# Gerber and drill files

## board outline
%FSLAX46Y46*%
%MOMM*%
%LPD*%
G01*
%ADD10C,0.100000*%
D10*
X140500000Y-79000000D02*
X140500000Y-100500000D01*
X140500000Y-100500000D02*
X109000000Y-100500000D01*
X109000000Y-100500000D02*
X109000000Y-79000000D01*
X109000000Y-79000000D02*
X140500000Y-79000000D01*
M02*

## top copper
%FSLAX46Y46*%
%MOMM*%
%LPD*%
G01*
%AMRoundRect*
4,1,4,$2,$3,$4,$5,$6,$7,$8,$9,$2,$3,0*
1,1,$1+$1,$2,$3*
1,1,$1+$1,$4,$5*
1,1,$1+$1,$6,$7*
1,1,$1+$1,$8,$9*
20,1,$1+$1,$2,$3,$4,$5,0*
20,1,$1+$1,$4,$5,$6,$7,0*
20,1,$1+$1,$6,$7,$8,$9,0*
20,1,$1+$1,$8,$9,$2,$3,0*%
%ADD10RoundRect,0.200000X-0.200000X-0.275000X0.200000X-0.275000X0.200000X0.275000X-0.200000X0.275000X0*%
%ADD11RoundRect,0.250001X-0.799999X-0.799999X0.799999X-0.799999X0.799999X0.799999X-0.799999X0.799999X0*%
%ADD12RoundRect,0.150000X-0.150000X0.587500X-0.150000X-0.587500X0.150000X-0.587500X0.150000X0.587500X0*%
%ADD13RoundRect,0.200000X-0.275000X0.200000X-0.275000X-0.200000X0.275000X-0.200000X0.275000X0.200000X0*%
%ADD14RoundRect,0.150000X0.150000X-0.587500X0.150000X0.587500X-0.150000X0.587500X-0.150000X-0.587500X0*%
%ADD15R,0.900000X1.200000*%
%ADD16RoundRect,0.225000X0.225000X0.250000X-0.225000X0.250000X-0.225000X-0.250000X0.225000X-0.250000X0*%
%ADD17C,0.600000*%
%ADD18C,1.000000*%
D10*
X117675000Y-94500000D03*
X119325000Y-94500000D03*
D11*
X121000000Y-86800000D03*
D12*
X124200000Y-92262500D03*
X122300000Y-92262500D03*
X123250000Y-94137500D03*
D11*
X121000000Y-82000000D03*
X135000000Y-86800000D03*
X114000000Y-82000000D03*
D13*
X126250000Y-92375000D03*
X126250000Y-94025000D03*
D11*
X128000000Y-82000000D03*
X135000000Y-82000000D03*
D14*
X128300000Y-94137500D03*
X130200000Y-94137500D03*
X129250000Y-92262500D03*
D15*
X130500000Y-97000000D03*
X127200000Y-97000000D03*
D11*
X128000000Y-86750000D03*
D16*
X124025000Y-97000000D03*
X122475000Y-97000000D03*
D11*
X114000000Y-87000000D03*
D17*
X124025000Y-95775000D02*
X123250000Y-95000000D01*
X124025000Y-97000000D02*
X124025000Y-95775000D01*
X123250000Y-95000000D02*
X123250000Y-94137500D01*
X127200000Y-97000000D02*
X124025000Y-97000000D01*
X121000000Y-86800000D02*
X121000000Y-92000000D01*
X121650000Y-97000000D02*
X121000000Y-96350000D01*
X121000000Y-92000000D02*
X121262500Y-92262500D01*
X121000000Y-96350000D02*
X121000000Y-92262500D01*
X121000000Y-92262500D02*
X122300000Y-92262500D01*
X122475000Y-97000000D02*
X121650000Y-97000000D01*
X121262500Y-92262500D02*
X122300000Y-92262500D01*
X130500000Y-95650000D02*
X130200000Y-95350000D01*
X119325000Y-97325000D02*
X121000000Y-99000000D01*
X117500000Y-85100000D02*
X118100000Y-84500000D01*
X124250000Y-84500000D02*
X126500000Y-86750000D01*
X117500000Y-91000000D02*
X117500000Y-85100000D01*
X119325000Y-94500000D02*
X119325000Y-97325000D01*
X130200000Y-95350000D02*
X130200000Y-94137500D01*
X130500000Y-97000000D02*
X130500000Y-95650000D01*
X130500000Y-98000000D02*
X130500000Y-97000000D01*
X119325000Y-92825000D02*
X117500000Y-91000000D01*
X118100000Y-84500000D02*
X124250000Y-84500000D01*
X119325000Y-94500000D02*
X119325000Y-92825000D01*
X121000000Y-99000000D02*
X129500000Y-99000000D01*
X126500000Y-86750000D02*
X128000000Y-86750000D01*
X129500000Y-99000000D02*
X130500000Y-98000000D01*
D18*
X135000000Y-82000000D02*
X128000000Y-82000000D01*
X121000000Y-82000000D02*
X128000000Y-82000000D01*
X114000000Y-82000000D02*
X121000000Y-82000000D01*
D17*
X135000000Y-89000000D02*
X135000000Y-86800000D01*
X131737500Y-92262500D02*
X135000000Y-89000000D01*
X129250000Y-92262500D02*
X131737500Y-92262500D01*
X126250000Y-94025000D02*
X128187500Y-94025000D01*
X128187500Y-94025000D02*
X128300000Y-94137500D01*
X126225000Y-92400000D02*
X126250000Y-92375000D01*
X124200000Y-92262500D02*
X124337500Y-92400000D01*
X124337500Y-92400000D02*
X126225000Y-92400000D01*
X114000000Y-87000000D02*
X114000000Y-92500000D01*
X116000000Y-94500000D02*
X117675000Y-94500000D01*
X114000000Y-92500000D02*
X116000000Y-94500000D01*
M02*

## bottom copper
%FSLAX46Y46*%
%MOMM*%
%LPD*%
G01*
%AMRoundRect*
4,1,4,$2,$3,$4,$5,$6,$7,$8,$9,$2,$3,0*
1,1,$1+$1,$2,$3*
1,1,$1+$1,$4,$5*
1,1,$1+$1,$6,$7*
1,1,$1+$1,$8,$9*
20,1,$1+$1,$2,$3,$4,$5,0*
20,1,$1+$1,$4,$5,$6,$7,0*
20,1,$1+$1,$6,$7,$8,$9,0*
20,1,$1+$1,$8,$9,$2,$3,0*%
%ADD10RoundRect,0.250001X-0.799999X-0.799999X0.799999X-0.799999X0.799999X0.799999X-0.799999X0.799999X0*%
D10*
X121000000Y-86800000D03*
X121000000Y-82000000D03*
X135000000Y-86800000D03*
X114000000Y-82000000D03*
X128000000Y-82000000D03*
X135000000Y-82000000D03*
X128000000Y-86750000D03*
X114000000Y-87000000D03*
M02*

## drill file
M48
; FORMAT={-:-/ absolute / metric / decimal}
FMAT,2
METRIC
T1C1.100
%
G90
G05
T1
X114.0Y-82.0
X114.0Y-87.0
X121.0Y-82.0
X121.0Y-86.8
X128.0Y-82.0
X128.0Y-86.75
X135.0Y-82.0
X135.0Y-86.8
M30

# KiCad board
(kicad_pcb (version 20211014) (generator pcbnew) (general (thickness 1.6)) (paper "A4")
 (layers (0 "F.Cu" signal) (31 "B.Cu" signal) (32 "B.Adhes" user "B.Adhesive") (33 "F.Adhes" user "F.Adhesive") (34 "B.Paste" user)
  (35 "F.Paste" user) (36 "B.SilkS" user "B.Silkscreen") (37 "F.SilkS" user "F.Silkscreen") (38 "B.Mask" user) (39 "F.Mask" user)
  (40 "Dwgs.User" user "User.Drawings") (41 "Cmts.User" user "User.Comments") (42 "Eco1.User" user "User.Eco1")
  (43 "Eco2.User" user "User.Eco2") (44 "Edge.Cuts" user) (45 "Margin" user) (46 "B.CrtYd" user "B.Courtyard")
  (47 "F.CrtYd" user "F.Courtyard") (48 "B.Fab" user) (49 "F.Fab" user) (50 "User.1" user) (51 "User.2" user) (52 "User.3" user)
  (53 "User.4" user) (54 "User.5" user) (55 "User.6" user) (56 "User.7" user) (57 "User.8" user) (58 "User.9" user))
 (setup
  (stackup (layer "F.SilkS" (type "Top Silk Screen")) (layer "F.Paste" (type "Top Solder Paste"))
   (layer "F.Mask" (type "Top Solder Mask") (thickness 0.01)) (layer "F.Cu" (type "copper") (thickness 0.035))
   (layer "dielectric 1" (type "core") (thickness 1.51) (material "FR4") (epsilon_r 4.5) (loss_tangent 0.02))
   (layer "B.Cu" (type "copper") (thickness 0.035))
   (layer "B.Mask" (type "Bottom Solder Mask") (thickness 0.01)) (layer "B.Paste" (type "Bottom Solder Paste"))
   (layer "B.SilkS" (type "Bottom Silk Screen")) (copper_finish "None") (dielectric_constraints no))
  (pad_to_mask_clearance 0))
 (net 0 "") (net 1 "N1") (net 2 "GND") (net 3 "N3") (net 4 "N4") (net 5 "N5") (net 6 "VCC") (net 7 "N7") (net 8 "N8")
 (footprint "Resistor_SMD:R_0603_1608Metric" (layer "F.Cu") (at 118.5 94.5)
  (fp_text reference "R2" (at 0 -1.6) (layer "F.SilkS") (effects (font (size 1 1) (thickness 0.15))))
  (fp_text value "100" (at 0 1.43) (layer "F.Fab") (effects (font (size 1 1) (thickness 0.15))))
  (pad "1" smd roundrect (at -0.825 0) (size 0.8 0.95) (layers "F.Cu" "F.Paste" "F.Mask") (roundrect_rratio 0.25) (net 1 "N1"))
  (pad "2" smd roundrect (at 0.825 0) (size 0.8 0.95) (layers "F.Cu" "F.Paste" "F.Mask") (roundrect_rratio 0.25) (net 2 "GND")))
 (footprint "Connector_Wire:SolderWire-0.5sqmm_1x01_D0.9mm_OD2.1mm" (layer "F.Cu") (at 121 86.8)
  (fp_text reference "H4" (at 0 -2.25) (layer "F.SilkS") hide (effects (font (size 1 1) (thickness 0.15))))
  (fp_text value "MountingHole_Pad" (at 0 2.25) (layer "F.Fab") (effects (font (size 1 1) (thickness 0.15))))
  (pad "1" thru_hole roundrect (at 0 0) (size 2.1 2.1) (drill 1.1) (layers *.Cu *.Mask) (roundrect_rratio 0.119048) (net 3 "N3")))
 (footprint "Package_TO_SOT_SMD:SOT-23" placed (layer "F.Cu") (at 123.25 93.2 -90)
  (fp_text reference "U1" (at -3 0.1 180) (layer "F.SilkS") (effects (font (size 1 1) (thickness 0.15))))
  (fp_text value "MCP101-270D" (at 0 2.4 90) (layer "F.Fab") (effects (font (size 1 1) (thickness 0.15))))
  (pad "1" smd roundrect (at -0.9375 -0.95 270) (size 1.475 0.6) (layers "F.Cu" "F.Paste" "F.Mask") (roundrect_rratio 0.25) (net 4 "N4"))
  (pad "2" smd roundrect (at -0.9375 0.95 270) (size 1.475 0.6) (layers "F.Cu" "F.Paste" "F.Mask") (roundrect_rratio 0.25) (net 3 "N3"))
  (pad "3" smd roundrect (at 0.9375 0 270) (size 1.475 0.6) (layers "F.Cu" "F.Paste" "F.Mask") (roundrect_rratio 0.25) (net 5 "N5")))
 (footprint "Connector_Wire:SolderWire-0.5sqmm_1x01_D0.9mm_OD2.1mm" (layer "F.Cu") (at 121 82)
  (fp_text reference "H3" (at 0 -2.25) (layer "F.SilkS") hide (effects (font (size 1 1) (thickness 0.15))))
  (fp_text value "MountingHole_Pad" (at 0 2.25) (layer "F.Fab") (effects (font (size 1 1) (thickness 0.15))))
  (pad "1" thru_hole roundrect (at 0 0) (size 2.1 2.1) (drill 1.1) (layers *.Cu *.Mask) (roundrect_rratio 0.119048) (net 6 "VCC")))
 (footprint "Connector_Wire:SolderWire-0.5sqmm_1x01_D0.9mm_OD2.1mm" (layer "F.Cu") (at 135 86.8)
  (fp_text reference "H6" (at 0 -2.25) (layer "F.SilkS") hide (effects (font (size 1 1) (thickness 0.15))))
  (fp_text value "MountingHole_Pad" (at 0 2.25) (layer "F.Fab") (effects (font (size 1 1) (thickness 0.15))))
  (pad "1" thru_hole roundrect (at 0 0) (size 2.1 2.1) (drill 1.1) (layers *.Cu *.Mask) (roundrect_rratio 0.119048) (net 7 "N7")))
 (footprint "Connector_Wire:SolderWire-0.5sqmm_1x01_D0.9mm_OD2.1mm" (layer "F.Cu") (at 114 82)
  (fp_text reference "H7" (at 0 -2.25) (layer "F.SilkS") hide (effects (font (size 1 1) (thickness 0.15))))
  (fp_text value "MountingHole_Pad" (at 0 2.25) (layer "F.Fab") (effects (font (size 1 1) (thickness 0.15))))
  (pad "1" thru_hole roundrect (at 0 0) (size 2.1 2.1) (drill 1.1) (layers *.Cu *.Mask) (roundrect_rratio 0.119048) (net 6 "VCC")))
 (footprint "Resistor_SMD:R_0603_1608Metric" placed (layer "F.Cu") (at 126.25 93.2 -90)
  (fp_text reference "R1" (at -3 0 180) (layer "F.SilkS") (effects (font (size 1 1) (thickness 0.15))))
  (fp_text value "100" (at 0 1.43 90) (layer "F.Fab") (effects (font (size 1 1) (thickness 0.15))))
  (pad "1" smd roundrect (at -0.825 0 270) (size 0.8 0.95) (layers "F.Cu" "F.Paste" "F.Mask") (roundrect_rratio 0.25) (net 4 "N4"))
  (pad "2" smd roundrect (at 0.825 0 270) (size 0.8 0.95) (layers "F.Cu" "F.Paste" "F.Mask") (roundrect_rratio 0.25) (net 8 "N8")))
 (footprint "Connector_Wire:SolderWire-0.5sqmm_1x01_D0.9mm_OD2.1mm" (layer "F.Cu") (at 128 82)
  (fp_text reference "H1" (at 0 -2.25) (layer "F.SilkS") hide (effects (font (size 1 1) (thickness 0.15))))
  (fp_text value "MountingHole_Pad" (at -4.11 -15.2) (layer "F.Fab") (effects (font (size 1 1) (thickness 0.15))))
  (pad "1" thru_hole roundrect (at 0 0) (size 2.1 2.1) (drill 1.1) (layers *.Cu *.Mask) (roundrect_rratio 0.119048) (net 6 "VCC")))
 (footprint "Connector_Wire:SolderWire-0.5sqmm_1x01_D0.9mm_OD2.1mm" (layer "F.Cu") (at 135 82)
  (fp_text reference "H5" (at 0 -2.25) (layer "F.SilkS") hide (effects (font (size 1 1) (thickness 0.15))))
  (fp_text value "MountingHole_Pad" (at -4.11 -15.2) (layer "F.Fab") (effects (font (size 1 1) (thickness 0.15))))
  (pad "1" thru_hole roundrect (at 0 0) (size 2.1 2.1) (drill 1.1) (layers *.Cu *.Mask) (roundrect_rratio 0.119048) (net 6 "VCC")))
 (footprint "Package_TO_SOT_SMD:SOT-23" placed (layer "F.Cu") (at 129.25 93.2 90)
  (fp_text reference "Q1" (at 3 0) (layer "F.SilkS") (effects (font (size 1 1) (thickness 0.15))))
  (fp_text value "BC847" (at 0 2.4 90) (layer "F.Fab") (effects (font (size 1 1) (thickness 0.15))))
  (pad "1" smd roundrect (at -0.9375 -0.95 90) (size 1.475 0.6) (layers "F.Cu" "F.Paste" "F.Mask") (roundrect_rratio 0.25) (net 8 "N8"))
  (pad "2" smd roundrect (at -0.9375 0.95 90) (size 1.475 0.6) (layers "F.Cu" "F.Paste" "F.Mask") (roundrect_rratio 0.25) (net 2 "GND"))
  (pad "3" smd roundrect (at 0.9375 0 90) (size 1.475 0.6) (layers "F.Cu" "F.Paste" "F.Mask") (roundrect_rratio 0.25) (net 7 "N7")))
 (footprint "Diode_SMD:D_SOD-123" (layer "F.Cu") (at 128.85 97 180)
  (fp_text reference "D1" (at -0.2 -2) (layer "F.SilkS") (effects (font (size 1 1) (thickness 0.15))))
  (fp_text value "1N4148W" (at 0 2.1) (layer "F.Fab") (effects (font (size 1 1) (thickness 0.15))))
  (pad "1" smd rect (at -1.65 0 180) (size 0.9 1.2) (layers "F.Cu" "F.Paste" "F.Mask") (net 2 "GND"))
  (pad "2" smd rect (at 1.65 0 180) (size 0.9 1.2) (layers "F.Cu" "F.Paste" "F.Mask") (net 5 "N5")))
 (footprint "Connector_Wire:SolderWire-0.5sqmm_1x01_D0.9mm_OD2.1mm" (layer "F.Cu") (at 128 86.75)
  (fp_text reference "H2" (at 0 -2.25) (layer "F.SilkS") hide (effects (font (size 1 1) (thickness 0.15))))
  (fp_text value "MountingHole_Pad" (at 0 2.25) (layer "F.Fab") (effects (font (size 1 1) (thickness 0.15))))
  (pad "1" thru_hole roundrect (at 0 0) (size 2.1 2.1) (drill 1.1) (layers *.Cu *.Mask) (roundrect_rratio 0.119048) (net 2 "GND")))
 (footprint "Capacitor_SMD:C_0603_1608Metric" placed (layer "F.Cu") (at 123.25 97 180)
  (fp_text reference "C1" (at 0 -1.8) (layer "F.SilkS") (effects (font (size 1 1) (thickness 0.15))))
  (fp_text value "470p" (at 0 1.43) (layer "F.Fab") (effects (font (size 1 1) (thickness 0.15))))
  (pad "1" smd roundrect (at -0.775 0 180) (size 0.9 0.95) (layers "F.Cu" "F.Paste" "F.Mask") (roundrect_rratio 0.25) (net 5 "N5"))
  (pad "2" smd roundrect (at 0.775 0 180) (size 0.9 0.95) (layers "F.Cu" "F.Paste" "F.Mask") (roundrect_rratio 0.25) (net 3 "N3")))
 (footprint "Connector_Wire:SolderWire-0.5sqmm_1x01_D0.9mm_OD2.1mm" (layer "F.Cu") (at 114 87)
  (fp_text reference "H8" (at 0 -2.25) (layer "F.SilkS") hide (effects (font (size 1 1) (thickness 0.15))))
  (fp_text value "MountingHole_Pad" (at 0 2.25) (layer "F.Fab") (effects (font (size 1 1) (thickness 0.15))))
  (pad "1" thru_hole roundrect (at 0 0) (size 2.1 2.1) (drill 1.1) (layers *.Cu *.Mask) (roundrect_rratio 0.119048) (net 1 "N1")))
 (gr_line (start 140.5 79) (end 140.5 100.5) (layer "Edge.Cuts") (width 0.1))
 (gr_line (start 140.5 100.5) (end 109 100.5) (layer "Edge.Cuts") (width 0.1))
 (gr_line (start 109 100.5) (end 109 79) (layer "Edge.Cuts") (width 0.1))
 (gr_line (start 109 79) (end 140.5 79) (layer "Edge.Cuts") (width 0.1))
 (segment (start 124.025 95.775) (end 123.25 95) (width 0.6) (layer "F.Cu") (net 5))
 (segment (start 124.025 97) (end 124.025 95.775) (width 0.6) (layer "F.Cu") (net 5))
 (segment (start 123.25 95) (end 123.25 94.1375) (width 0.6) (layer "F.Cu") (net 5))
 (segment (start 127.2 97) (end 124.025 97) (width 0.6) (layer "F.Cu") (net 5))
 (segment (start 121 86.8) (end 121 92) (width 0.6) (layer "F.Cu") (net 3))
 (segment (start 121.65 97) (end 121 96.35) (width 0.6) (layer "F.Cu") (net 3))
 (segment (start 121 92) (end 121.2625 92.2625) (width 0.6) (layer "F.Cu") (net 3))
 (segment (start 121 96.35) (end 121 92.2625) (width 0.6) (layer "F.Cu") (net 3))
 (segment (start 121 92.2625) (end 122.3 92.2625) (width 0.6) (layer "F.Cu") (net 3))
 (segment (start 122.475 97) (end 121.65 97) (width 0.6) (layer "F.Cu") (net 3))
 (segment (start 121.2625 92.2625) (end 122.3 92.2625) (width 0.6) (layer "F.Cu") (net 3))
 (segment (start 130.5 95.65) (end 130.2 95.35) (width 0.6) (layer "F.Cu") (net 2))
 (segment (start 119.325 97.325) (end 121 99) (width 0.6) (layer "F.Cu") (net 2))
 (segment (start 117.5 85.1) (end 118.1 84.5) (width 0.6) (layer "F.Cu") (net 2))
 (segment (start 124.25 84.5) (end 126.5 86.75) (width 0.6) (layer "F.Cu") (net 2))
 (segment (start 117.5 91) (end 117.5 85.1) (width 0.6) (layer "F.Cu") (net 2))
 (segment (start 119.325 94.5) (end 119.325 97.325) (width 0.6) (layer "F.Cu") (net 2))
 (segment (start 130.2 95.35) (end 130.2 94.1375) (width 0.6) (layer "F.Cu") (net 2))
 (segment (start 130.5 97) (end 130.5 95.65) (width 0.6) (layer "F.Cu") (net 2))
 (segment (start 130.5 98) (end 130.5 97) (width 0.6) (layer "F.Cu") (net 2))
 (segment (start 119.325 92.825) (end 117.5 91) (width 0.6) (layer "F.Cu") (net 2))
 (segment (start 118.1 84.5) (end 124.25 84.5) (width 0.6) (layer "F.Cu") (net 2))
 (segment (start 119.325 94.5) (end 119.325 92.825) (width 0.6) (layer "F.Cu") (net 2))
 (segment (start 121 99) (end 129.5 99) (width 0.6) (layer "F.Cu") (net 2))
 (segment (start 126.5 86.75) (end 128 86.75) (width 0.6) (layer "F.Cu") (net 2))
 (segment (start 129.5 99) (end 130.5 98) (width 0.6) (layer "F.Cu") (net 2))
 (segment (start 135 82) (end 128 82) (width 1) (layer "F.Cu") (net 6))
 (segment (start 121 82) (end 128 82) (width 1) (layer "F.Cu") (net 6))
 (segment (start 114 82) (end 121 82) (width 1) (layer "F.Cu") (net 6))
 (segment (start 135 89) (end 135 86.8) (width 0.6) (layer "F.Cu") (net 7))
 (segment (start 131.7375 92.2625) (end 135 89) (width 0.6) (layer "F.Cu") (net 7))
 (segment (start 129.25 92.2625) (end 131.7375 92.2625) (width 0.6) (layer "F.Cu") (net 7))
 (segment (start 126.25 94.025) (end 128.1875 94.025) (width 0.6) (layer "F.Cu") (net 8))
 (segment (start 128.1875 94.025) (end 128.3 94.1375) (width 0.6) (layer "F.Cu") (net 8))
 (segment (start 126.225 92.4) (end 126.25 92.375) (width 0.6) (layer "F.Cu") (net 4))
 (segment (start 124.2 92.2625) (end 124.3375 92.4) (width 0.6) (layer "F.Cu") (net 4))
 (segment (start 124.3375 92.4) (end 126.225 92.4) (width 0.6) (layer "F.Cu") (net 4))
 (segment (start 114 87) (end 114 92.5) (width 0.6) (layer "F.Cu") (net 1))
 (segment (start 116 94.5) (end 117.675 94.5) (width 0.6) (layer "F.Cu") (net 1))
 (segment (start 114 92.5) (end 116 94.5) (width 0.6) (layer "F.Cu") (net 1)))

